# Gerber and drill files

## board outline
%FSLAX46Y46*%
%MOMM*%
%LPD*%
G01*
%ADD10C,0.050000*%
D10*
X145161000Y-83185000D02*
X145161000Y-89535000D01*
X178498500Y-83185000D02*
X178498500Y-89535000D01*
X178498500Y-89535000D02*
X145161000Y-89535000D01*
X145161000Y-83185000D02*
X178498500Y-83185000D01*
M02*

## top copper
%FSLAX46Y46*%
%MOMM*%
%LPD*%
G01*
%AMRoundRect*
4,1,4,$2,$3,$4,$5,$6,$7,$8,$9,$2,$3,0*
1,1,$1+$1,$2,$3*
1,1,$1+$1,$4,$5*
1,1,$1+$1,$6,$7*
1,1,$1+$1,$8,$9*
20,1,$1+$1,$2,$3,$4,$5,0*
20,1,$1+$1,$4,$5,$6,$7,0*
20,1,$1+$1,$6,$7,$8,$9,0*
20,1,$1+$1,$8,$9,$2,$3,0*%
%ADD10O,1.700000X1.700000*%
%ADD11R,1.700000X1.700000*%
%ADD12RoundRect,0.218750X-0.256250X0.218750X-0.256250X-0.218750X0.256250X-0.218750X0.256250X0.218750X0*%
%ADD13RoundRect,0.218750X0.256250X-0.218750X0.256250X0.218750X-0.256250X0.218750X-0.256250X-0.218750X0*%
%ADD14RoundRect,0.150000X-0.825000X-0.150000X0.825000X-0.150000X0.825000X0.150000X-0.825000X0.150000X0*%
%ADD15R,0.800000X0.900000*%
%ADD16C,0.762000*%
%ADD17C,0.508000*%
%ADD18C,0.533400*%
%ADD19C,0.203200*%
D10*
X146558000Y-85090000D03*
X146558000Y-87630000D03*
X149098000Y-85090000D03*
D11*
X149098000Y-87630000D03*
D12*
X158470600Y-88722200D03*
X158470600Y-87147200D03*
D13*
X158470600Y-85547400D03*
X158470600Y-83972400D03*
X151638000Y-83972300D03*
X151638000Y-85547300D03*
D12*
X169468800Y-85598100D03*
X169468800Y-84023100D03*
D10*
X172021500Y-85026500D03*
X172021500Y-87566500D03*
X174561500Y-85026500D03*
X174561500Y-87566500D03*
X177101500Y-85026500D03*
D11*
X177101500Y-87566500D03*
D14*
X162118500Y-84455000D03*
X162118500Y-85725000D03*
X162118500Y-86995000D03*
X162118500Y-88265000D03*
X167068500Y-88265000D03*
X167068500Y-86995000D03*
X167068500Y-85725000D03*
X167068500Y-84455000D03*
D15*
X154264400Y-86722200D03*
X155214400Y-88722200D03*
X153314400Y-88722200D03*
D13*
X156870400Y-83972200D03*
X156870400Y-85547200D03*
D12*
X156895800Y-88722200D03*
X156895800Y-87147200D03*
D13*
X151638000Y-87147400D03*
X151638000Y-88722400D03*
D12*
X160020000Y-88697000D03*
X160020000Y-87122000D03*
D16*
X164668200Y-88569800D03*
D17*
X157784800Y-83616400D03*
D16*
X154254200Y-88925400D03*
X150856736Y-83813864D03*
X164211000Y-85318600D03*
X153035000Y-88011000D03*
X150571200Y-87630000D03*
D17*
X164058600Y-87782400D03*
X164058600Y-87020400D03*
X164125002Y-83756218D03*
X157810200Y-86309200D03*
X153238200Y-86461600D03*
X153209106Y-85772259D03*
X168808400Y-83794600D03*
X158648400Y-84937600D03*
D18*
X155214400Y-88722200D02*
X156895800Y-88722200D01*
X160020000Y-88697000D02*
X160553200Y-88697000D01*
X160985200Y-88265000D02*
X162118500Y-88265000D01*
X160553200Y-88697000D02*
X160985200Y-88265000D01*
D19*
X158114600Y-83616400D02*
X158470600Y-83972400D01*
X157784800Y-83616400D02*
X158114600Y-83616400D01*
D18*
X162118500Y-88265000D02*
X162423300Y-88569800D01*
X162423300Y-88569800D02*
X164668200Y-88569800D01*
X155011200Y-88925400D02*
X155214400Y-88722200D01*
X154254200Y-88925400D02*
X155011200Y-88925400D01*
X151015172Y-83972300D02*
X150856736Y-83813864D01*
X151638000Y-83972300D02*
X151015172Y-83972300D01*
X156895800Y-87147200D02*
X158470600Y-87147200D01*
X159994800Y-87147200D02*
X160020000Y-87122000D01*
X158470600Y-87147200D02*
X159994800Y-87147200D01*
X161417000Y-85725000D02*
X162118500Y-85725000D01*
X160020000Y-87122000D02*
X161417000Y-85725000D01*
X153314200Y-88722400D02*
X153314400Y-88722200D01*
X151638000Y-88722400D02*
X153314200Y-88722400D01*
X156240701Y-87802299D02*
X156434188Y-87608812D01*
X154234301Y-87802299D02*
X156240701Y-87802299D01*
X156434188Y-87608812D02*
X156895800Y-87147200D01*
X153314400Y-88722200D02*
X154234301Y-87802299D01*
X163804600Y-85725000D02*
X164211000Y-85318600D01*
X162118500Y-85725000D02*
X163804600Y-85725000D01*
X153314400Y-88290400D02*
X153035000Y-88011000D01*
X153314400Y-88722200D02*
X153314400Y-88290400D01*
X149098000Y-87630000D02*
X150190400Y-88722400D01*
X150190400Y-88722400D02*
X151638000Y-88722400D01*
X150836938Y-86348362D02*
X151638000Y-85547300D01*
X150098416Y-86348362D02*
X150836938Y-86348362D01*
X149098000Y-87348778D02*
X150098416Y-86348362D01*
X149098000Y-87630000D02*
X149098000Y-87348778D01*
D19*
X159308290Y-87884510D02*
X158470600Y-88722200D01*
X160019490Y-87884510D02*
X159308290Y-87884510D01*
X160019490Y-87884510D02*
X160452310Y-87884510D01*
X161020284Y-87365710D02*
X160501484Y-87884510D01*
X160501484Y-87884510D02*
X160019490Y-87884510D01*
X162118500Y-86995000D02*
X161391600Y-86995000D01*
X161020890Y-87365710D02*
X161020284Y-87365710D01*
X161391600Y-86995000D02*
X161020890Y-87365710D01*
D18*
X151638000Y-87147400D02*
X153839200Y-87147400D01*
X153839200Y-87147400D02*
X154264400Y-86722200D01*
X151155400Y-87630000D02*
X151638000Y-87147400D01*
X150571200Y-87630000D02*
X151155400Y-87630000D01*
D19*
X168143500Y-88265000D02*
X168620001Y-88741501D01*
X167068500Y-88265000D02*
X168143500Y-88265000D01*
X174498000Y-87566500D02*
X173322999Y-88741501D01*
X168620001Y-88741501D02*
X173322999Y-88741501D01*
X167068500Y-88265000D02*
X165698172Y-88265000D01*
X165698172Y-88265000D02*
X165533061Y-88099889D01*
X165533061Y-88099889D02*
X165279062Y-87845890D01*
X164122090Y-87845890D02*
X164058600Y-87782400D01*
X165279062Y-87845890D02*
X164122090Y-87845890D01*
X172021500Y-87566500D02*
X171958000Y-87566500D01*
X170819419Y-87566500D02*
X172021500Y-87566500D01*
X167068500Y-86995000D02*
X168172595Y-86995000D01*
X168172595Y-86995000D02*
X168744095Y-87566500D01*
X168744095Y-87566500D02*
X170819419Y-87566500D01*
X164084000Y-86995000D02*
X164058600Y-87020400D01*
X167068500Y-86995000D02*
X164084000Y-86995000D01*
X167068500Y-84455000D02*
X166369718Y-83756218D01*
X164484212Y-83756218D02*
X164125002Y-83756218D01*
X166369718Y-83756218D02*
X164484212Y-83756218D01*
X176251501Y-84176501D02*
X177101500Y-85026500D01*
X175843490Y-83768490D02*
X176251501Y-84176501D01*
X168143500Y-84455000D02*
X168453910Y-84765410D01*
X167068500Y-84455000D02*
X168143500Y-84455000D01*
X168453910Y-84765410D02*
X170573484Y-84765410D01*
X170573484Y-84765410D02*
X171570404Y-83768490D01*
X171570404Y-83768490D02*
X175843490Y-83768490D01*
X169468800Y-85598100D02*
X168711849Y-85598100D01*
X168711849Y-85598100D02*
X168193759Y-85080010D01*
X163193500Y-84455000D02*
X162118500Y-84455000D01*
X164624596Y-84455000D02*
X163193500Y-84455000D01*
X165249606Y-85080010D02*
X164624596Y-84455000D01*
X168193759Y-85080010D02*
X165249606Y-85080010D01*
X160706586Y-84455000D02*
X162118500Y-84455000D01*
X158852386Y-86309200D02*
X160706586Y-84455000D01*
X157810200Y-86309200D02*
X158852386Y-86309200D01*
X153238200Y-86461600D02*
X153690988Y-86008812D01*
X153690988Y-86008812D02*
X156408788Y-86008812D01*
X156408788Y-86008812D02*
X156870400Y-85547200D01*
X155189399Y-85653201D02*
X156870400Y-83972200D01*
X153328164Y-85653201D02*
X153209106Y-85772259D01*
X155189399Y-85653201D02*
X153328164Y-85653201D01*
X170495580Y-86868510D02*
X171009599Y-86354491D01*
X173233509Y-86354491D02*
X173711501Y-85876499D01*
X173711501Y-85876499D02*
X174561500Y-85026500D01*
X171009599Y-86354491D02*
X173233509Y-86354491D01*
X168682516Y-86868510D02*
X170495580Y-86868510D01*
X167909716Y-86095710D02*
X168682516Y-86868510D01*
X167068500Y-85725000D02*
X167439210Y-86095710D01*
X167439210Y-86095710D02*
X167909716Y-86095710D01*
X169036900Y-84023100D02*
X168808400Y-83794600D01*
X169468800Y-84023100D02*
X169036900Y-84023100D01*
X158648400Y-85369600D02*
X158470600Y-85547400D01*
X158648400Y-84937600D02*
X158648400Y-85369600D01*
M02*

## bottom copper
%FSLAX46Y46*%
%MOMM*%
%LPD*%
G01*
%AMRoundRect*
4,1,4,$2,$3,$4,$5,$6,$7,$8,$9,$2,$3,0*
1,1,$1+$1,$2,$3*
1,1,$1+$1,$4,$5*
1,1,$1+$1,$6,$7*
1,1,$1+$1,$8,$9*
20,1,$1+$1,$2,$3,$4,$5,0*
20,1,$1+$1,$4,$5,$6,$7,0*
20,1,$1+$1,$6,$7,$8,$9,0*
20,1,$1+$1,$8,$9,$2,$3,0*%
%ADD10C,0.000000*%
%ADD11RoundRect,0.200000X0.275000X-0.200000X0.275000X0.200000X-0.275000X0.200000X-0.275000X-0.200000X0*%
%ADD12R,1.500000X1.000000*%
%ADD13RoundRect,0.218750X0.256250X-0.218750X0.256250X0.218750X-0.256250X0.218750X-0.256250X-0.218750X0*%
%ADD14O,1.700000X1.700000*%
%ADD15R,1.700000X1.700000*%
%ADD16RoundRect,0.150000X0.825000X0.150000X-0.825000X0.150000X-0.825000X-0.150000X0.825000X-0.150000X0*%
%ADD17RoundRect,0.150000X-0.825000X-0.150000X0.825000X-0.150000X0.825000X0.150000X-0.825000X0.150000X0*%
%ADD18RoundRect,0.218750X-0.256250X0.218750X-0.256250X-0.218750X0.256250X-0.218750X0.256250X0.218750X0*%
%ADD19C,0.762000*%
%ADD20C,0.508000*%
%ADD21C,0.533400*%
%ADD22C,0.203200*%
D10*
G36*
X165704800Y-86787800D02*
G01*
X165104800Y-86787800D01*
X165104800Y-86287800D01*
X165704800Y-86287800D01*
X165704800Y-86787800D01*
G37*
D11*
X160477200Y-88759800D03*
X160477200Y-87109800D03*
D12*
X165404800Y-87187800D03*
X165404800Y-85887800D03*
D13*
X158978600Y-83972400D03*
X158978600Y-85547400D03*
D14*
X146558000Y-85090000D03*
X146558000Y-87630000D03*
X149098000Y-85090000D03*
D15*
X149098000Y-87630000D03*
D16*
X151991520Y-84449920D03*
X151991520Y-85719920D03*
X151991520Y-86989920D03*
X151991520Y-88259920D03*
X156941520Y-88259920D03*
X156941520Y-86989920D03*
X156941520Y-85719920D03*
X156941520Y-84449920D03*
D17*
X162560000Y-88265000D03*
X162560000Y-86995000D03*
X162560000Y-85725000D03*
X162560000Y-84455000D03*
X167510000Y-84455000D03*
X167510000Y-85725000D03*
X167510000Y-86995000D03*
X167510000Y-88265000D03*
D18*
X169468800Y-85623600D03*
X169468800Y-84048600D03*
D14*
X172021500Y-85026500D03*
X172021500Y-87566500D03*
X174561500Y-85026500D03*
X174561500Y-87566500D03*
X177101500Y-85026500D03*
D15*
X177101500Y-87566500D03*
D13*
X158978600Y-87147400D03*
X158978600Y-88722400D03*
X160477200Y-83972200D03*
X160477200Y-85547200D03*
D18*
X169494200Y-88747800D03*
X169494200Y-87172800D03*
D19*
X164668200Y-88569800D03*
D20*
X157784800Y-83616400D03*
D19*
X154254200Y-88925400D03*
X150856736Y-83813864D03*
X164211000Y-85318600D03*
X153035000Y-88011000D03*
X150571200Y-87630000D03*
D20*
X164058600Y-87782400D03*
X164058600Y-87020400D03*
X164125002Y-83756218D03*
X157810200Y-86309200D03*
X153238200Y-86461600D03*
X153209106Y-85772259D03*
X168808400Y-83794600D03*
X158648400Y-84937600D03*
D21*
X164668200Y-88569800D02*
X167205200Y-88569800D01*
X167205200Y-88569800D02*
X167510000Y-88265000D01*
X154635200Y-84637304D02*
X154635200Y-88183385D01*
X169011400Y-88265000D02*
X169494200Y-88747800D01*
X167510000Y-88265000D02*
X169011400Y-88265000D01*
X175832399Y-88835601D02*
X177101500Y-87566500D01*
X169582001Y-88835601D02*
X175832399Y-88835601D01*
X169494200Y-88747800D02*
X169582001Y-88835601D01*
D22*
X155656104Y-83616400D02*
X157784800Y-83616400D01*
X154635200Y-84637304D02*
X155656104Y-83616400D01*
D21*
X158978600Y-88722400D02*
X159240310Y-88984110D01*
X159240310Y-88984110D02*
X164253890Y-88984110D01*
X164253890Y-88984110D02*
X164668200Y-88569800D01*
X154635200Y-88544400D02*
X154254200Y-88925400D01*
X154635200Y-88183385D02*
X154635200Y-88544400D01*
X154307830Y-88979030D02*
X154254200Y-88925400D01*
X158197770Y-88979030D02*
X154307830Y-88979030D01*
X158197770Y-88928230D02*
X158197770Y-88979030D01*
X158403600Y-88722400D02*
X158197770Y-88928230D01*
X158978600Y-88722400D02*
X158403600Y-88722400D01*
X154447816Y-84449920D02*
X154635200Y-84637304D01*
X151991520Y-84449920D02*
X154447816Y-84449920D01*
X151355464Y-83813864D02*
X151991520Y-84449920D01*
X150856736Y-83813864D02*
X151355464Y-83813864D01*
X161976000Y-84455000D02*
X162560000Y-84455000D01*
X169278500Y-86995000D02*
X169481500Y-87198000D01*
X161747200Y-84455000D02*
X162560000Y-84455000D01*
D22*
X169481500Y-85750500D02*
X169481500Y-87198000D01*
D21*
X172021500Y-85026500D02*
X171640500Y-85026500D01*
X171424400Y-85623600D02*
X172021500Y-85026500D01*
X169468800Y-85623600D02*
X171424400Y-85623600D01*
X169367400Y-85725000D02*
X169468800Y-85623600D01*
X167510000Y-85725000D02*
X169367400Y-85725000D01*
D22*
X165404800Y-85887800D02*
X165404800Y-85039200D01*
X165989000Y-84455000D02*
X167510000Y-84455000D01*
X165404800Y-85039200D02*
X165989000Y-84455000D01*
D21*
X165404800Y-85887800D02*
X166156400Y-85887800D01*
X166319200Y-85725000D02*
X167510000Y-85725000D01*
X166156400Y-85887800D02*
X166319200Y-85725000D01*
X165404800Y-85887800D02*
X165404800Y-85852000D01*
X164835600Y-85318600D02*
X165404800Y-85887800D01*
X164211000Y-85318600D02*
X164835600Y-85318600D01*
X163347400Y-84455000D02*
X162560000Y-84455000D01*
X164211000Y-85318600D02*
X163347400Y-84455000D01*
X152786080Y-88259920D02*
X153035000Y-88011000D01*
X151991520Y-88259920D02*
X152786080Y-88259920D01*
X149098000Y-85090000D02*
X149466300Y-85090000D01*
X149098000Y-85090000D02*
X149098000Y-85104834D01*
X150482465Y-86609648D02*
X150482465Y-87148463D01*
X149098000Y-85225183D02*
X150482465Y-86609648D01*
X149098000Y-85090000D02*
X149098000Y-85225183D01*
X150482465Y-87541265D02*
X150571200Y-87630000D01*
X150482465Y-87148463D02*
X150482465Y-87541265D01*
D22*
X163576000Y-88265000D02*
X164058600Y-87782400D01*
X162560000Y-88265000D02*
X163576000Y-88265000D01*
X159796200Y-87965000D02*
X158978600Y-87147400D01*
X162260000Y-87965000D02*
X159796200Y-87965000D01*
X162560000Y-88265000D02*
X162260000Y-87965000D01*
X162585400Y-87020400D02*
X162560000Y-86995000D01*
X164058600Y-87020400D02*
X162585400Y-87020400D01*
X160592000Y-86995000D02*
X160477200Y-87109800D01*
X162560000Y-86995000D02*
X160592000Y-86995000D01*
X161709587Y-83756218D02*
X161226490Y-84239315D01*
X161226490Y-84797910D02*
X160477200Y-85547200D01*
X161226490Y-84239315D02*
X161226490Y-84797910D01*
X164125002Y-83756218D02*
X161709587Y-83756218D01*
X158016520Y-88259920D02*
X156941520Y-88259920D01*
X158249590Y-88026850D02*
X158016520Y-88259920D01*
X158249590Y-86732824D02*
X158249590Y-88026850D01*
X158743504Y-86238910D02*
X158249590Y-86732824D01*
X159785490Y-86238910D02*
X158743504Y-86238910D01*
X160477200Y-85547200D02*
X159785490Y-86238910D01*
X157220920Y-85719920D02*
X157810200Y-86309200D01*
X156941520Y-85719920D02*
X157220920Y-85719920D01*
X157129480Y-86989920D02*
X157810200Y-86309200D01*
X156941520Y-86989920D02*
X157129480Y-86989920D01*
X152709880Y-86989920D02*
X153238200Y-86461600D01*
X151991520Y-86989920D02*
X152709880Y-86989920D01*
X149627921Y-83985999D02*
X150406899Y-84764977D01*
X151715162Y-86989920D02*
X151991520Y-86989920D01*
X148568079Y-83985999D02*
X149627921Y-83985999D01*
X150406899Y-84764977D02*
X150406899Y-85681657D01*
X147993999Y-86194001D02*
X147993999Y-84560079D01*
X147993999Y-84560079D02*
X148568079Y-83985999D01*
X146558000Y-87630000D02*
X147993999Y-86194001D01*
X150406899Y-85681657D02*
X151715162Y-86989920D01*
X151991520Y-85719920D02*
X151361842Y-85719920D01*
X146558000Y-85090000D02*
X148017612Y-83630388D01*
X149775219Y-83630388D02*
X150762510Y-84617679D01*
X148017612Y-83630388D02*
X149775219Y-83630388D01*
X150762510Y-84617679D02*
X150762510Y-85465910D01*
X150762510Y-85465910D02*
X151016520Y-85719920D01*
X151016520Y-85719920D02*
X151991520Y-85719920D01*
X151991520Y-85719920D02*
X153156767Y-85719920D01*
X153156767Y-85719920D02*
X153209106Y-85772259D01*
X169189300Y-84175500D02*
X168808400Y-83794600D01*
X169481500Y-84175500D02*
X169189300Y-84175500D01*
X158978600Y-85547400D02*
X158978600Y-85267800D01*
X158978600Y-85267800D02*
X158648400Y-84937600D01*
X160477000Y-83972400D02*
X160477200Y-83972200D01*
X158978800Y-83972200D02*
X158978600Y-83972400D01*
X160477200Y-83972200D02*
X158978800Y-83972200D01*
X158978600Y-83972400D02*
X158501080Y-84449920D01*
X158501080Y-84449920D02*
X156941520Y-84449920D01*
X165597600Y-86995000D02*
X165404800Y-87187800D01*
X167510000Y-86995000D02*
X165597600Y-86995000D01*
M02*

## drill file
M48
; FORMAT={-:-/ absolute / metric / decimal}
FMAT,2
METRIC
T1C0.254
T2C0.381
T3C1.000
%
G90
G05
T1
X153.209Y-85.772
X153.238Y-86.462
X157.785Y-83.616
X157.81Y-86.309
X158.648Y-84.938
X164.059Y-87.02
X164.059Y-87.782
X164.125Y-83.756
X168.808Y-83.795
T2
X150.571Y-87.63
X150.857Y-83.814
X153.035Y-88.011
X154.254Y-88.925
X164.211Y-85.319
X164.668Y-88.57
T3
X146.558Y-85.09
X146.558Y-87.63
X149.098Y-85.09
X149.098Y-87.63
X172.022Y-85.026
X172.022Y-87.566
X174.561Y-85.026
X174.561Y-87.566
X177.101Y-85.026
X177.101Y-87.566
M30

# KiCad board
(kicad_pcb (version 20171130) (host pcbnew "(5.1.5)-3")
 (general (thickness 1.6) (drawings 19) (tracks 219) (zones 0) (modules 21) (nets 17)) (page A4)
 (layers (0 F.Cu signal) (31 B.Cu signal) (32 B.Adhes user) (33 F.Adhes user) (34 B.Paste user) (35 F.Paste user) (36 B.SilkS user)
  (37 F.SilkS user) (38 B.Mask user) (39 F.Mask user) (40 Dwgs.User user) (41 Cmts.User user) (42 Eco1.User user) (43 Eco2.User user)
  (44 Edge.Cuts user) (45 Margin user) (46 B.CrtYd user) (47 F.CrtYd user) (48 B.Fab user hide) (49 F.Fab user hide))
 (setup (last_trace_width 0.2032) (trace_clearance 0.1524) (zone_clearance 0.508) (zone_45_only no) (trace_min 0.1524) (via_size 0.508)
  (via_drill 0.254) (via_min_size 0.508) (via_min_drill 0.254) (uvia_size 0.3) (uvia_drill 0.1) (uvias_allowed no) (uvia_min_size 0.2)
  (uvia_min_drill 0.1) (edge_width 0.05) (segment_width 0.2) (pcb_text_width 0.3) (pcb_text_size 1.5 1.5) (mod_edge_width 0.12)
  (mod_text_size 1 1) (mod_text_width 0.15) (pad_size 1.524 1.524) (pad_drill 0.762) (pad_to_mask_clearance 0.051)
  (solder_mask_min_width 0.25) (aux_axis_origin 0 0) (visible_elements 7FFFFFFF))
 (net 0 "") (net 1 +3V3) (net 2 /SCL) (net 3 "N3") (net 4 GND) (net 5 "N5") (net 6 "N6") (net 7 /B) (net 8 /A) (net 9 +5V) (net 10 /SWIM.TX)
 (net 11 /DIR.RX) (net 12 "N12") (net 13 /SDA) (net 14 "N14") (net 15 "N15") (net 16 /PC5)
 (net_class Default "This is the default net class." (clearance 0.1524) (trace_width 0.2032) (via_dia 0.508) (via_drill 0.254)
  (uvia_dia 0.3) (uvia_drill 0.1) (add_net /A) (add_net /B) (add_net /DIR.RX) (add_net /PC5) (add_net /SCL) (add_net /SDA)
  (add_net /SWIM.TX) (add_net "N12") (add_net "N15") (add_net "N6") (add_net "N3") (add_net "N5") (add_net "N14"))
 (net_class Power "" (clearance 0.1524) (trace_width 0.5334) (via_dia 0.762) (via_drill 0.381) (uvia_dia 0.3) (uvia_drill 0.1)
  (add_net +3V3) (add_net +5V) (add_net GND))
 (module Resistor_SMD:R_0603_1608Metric (layer B.Cu) (at 160.4772 87.9348 90)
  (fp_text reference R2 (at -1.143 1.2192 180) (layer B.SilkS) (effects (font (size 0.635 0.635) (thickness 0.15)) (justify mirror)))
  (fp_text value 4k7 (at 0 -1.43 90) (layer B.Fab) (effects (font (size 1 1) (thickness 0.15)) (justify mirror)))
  (pad 1 smd roundrect (at -0.825 0 90) (size 0.8 0.95) (layers B.Cu B.Paste B.Mask) (roundrect_rratio 0.25) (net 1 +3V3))
  (pad 2 smd roundrect (at 0.825 0 90) (size 0.8 0.95) (layers B.Cu B.Paste B.Mask) (roundrect_rratio 0.25) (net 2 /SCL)))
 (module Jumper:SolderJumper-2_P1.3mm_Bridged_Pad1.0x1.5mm (layer B.Cu) (at 165.4048 86.5378 270)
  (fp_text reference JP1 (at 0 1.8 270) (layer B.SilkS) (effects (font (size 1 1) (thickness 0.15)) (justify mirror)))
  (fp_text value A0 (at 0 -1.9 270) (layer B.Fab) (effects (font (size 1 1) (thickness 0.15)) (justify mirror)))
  (fp_poly (pts (xy -0.25 0.3) (xy 0.25 0.3) (xy 0.25 -0.3) (xy -0.25 -0.3)) (layer B.Cu) (width 0))
  (pad 2 smd rect (at 0.65 0 270) (size 1 1.5) (layers B.Cu B.Mask) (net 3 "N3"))
  (pad 1 smd rect (at -0.65 0 270) (size 1 1.5) (layers B.Cu B.Mask) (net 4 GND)))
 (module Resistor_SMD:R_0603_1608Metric (layer B.Cu) (at 158.9786 84.7599 90)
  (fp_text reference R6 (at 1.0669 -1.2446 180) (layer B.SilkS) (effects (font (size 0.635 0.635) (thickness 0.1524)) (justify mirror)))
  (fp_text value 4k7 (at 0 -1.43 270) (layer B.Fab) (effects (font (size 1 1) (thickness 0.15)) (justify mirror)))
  (pad 2 smd roundrect (at 0.7875 0 90) (size 0.875 0.95) (layers B.Cu B.Paste B.Mask) (roundrect_rratio 0.25) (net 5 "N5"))
  (pad 1 smd roundrect (at -0.7875 0 90) (size 0.875 0.95) (layers B.Cu B.Paste B.Mask) (roundrect_rratio 0.25) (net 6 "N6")))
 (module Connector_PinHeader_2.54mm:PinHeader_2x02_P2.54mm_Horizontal (layer B.Cu) (at 149.098 87.63 90)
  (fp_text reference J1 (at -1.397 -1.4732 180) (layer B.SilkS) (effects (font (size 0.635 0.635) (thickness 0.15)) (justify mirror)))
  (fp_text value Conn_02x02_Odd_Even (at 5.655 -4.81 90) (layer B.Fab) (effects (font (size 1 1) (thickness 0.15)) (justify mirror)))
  (pad 4 thru_hole oval (at 2.54 -2.54 90) (size 1.7 1.7) (drill 1) (layers *.Cu *.Mask) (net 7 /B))
  (pad 3 thru_hole oval (at 0 -2.54 90) (size 1.7 1.7) (drill 1) (layers *.Cu *.Mask) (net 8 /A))
  (pad 2 thru_hole oval (at 2.54 0 90) (size 1.7 1.7) (drill 1) (layers *.Cu *.Mask) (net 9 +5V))
  (pad 1 thru_hole rect (at 0 0 90) (size 1.7 1.7) (drill 1) (layers *.Cu *.Mask) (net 4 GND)))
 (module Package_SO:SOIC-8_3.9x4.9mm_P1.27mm (layer B.Cu) (at 154.46652 86.35492 180)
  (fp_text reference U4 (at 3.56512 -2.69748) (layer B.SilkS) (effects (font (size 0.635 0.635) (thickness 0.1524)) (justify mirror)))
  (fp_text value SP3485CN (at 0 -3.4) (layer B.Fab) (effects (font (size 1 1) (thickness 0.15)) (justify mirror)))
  (pad 8 smd roundrect (at 2.475 1.905 180) (size 1.95 0.6) (layers B.Cu B.Paste B.Mask) (roundrect_rratio 0.25) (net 1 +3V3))
  (pad 7 smd roundrect (at 2.475 0.635 180) (size 1.95 0.6) (layers B.Cu B.Paste B.Mask) (roundrect_rratio 0.25) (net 7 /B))
  (pad 6 smd roundrect (at 2.475 -0.635 180) (size 1.95 0.6) (layers B.Cu B.Paste B.Mask) (roundrect_rratio 0.25) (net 8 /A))
  (pad 5 smd roundrect (at 2.475 -1.905 180) (size 1.95 0.6) (layers B.Cu B.Paste B.Mask) (roundrect_rratio 0.25) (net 4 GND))
  (pad 4 smd roundrect (at -2.475 -1.905 180) (size 1.95 0.6) (layers B.Cu B.Paste B.Mask) (roundrect_rratio 0.25) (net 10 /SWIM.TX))
  (pad 3 smd roundrect (at -2.475 -0.635 180) (size 1.95 0.6) (layers B.Cu B.Paste B.Mask) (roundrect_rratio 0.25) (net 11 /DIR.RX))
  (pad 2 smd roundrect (at -2.475 0.635 180) (size 1.95 0.6) (layers B.Cu B.Paste B.Mask) (roundrect_rratio 0.25) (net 11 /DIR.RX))
  (pad 1 smd roundrect (at -2.475 1.905 180) (size 1.95 0.6) (layers B.Cu B.Paste B.Mask) (roundrect_rratio 0.25) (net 5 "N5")))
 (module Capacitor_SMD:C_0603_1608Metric (layer F.Cu) (at 158.4706 87.9347 270)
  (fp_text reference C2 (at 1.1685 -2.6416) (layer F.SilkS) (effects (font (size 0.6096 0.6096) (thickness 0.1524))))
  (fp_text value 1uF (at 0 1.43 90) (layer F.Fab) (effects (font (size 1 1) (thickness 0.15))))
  (pad 2 smd roundrect (at 0.7875 0 270) (size 0.875 0.95) (layers F.Cu F.Paste F.Mask) (roundrect_rratio 0.25) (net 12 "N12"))
  (pad 1 smd roundrect (at -0.7875 0 270) (size 0.875 0.95) (layers F.Cu F.Paste F.Mask) (roundrect_rratio 0.25) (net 4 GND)))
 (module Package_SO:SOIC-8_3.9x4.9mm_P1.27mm (layer B.Cu) (at 165.035 86.36)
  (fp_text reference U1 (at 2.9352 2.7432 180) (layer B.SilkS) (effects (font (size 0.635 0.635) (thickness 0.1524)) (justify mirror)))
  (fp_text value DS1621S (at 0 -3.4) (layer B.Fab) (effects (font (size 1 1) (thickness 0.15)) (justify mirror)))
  (pad 1 smd roundrect (at -2.475 1.905) (size 1.95 0.6) (layers B.Cu B.Paste B.Mask) (roundrect_rratio 0.25) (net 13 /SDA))
  (pad 2 smd roundrect (at -2.475 0.635) (size 1.95 0.6) (layers B.Cu B.Paste B.Mask) (roundrect_rratio 0.25) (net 2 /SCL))
  (pad 3 smd roundrect (at -2.475 -0.635) (size 1.95 0.6) (layers B.Cu B.Paste B.Mask) (roundrect_rratio 0.25) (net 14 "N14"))
  (pad 4 smd roundrect (at -2.475 -1.905) (size 1.95 0.6) (layers B.Cu B.Paste B.Mask) (roundrect_rratio 0.25) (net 4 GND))
  (pad 5 smd roundrect (at 2.475 -1.905) (size 1.95 0.6) (layers B.Cu B.Paste B.Mask) (roundrect_rratio 0.25) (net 4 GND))
  (pad 6 smd roundrect (at 2.475 -0.635) (size 1.95 0.6) (layers B.Cu B.Paste B.Mask) (roundrect_rratio 0.25) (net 4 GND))
  (pad 7 smd roundrect (at 2.475 0.635) (size 1.95 0.6) (layers B.Cu B.Paste B.Mask) (roundrect_rratio 0.25) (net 3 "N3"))
  (pad 8 smd roundrect (at 2.475 1.905) (size 1.95 0.6) (layers B.Cu B.Paste B.Mask) (roundrect_rratio 0.25) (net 1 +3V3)))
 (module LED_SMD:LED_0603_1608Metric (layer F.Cu) (at 158.4706 84.7599 90)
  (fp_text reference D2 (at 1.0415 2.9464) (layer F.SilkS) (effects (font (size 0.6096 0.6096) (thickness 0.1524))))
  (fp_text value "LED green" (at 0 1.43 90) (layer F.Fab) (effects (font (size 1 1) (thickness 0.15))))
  (pad 1 smd roundrect (at -0.7875 0 90) (size 0.875 0.95) (layers F.Cu F.Paste F.Mask) (roundrect_rratio 0.25) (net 6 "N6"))
  (pad 2 smd roundrect (at 0.7875 0 90) (size 0.875 0.95) (layers F.Cu F.Paste F.Mask) (roundrect_rratio 0.25) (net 1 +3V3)))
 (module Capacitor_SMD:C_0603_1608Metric (layer F.Cu) (at 151.638 84.7598 90)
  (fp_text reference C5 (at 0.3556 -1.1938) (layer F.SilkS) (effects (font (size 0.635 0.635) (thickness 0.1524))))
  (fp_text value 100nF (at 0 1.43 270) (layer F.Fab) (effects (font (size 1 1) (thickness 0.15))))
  (pad 2 smd roundrect (at 0.7875 0 90) (size 0.875 0.95) (layers F.Cu F.Paste F.Mask) (roundrect_rratio 0.25) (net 1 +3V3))
  (pad 1 smd roundrect (at -0.7875 0 90) (size 0.875 0.95) (layers F.Cu F.Paste F.Mask) (roundrect_rratio 0.25) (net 4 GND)))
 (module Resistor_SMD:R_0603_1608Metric (layer B.Cu) (at 169.4688 84.8361 270)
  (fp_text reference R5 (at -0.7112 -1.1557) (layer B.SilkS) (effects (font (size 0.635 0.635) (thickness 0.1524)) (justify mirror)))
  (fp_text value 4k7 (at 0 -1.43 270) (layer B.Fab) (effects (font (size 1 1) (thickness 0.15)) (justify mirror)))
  (pad 2 smd roundrect (at 0.7875 0 270) (size 0.875 0.95) (layers B.Cu B.Paste B.Mask) (roundrect_rratio 0.25) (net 4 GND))
  (pad 1 smd roundrect (at -0.7875 0 270) (size 0.875 0.95) (layers B.Cu B.Paste B.Mask) (roundrect_rratio 0.25) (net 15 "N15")))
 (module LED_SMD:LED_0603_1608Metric (layer F.Cu) (at 169.4688 84.8106 270)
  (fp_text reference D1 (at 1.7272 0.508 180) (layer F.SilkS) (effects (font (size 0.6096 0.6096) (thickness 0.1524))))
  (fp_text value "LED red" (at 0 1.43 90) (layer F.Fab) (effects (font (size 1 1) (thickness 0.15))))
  (pad 2 smd roundrect (at 0.7875 0 270) (size 0.875 0.95) (layers F.Cu F.Paste F.Mask) (roundrect_rratio 0.25) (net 11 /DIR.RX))
  (pad 1 smd roundrect (at -0.7875 0 270) (size 0.875 0.95) (layers F.Cu F.Paste F.Mask) (roundrect_rratio 0.25) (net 15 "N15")))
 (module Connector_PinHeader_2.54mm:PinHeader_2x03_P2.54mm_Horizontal (layer B.Cu) (at 177.1015 87.5665 90)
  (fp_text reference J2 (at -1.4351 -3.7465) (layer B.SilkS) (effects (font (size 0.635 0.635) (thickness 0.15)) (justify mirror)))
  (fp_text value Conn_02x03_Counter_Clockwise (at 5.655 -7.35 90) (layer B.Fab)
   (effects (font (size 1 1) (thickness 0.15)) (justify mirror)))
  (pad 6 thru_hole oval (at 2.54 -5.08 90) (size 1.7 1.7) (drill 1) (layers *.Cu *.Mask) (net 4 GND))
  (pad 5 thru_hole oval (at 0 -5.08 90) (size 1.7 1.7) (drill 1) (layers *.Cu *.Mask) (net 2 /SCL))
  (pad 4 thru_hole oval (at 2.54 -2.54 90) (size 1.7 1.7) (drill 1) (layers *.Cu *.Mask) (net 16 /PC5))
  (pad 3 thru_hole oval (at 0 -2.54 90) (size 1.7 1.7) (drill 1) (layers *.Cu *.Mask) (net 13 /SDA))
  (pad 2 thru_hole oval (at 2.54 0 90) (size 1.7 1.7) (drill 1) (layers *.Cu *.Mask) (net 10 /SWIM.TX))
  (pad 1 thru_hole rect (at 0 0 90) (size 1.7 1.7) (drill 1) (layers *.Cu *.Mask) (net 1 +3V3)))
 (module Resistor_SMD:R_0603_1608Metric (layer B.Cu) (at 158.9786 87.9349 90)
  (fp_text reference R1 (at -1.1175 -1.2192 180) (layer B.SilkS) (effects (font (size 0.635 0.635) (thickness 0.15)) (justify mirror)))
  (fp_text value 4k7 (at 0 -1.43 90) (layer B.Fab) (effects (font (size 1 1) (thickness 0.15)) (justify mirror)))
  (pad 2 smd roundrect (at 0.7875 0 90) (size 0.875 0.95) (layers B.Cu B.Paste B.Mask) (roundrect_rratio 0.25) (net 13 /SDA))
  (pad 1 smd roundrect (at -0.7875 0 90) (size 0.875 0.95) (layers B.Cu B.Paste B.Mask) (roundrect_rratio 0.25) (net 1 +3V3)))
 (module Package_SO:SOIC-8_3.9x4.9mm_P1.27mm (layer F.Cu) (at 164.5935 86.36)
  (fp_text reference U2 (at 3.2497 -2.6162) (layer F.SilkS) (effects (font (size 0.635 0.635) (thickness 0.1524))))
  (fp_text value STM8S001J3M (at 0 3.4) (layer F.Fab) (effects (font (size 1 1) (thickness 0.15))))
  (pad 1 smd roundrect (at -2.475 -1.905) (size 1.95 0.6) (layers F.Cu F.Paste F.Mask) (roundrect_rratio 0.25) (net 11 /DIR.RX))
  (pad 2 smd roundrect (at -2.475 -0.635) (size 1.95 0.6) (layers F.Cu F.Paste F.Mask) (roundrect_rratio 0.25) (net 4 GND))
  (pad 3 smd roundrect (at -2.475 0.635) (size 1.95 0.6) (layers F.Cu F.Paste F.Mask) (roundrect_rratio 0.25) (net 12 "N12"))
  (pad 4 smd roundrect (at -2.475 1.905) (size 1.95 0.6) (layers F.Cu F.Paste F.Mask) (roundrect_rratio 0.25) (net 1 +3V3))
  (pad 5 smd roundrect (at 2.475 1.905) (size 1.95 0.6) (layers F.Cu F.Paste F.Mask) (roundrect_rratio 0.25) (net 13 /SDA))
  (pad 6 smd roundrect (at 2.475 0.635) (size 1.95 0.6) (layers F.Cu F.Paste F.Mask) (roundrect_rratio 0.25) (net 2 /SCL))
  (pad 7 smd roundrect (at 2.475 -0.635) (size 1.95 0.6) (layers F.Cu F.Paste F.Mask) (roundrect_rratio 0.25) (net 16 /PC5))
  (pad 8 smd roundrect (at 2.475 -1.905) (size 1.95 0.6) (layers F.Cu F.Paste F.Mask) (roundrect_rratio 0.25) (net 10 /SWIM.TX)))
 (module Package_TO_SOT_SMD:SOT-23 (layer F.Cu) (at 154.2644 87.7222 90)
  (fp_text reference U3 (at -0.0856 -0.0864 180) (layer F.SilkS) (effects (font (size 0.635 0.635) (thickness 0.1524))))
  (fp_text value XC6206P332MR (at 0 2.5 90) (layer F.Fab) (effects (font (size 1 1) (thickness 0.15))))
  (pad 3 smd rect (at 1 0 90) (size 0.9 0.8) (layers F.Cu F.Paste F.Mask) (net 9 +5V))
  (pad 2 smd rect (at -1 0.95 90) (size 0.9 0.8) (layers F.Cu F.Paste F.Mask) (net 1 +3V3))
  (pad 1 smd rect (at -1 -0.95 90) (size 0.9 0.8) (layers F.Cu F.Paste F.Mask) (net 4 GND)))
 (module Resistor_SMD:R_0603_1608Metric (layer F.Cu) (at 156.8704 84.7597 90)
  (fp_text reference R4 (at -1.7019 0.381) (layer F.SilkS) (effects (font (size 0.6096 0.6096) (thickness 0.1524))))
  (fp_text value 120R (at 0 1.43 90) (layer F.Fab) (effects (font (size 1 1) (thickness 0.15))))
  (pad 2 smd roundrect (at 0.7875 0 90) (size 0.875 0.95) (layers F.Cu F.Paste F.Mask) (roundrect_rratio 0.25) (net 7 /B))
  (pad 1 smd roundrect (at -0.7875 0 90) (size 0.875 0.95) (layers F.Cu F.Paste F.Mask) (roundrect_rratio 0.25) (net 8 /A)))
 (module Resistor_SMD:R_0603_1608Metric (layer B.Cu) (at 160.4772 84.7597 90)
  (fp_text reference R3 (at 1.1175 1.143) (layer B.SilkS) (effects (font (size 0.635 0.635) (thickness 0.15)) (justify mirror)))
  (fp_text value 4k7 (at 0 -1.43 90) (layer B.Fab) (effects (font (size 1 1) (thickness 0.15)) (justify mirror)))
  (pad 2 smd roundrect (at 0.7875 0 90) (size 0.875 0.95) (layers B.Cu B.Paste B.Mask) (roundrect_rratio 0.25) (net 5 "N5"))
  (pad 1 smd roundrect (at -0.7875 0 90) (size 0.875 0.95) (layers B.Cu B.Paste B.Mask) (roundrect_rratio 0.25) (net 10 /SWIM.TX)))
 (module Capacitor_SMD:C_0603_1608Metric (layer F.Cu) (at 156.8958 87.9347 270)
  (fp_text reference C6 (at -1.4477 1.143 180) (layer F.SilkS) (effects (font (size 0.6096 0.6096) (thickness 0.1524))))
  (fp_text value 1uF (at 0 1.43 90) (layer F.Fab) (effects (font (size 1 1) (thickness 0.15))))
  (pad 2 smd roundrect (at 0.7875 0 270) (size 0.875 0.95) (layers F.Cu F.Paste F.Mask) (roundrect_rratio 0.25) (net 1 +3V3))
  (pad 1 smd roundrect (at -0.7875 0 270) (size 0.875 0.95) (layers F.Cu F.Paste F.Mask) (roundrect_rratio 0.25) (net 4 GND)))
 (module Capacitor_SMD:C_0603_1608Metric (layer F.Cu) (at 151.638 87.9349 90)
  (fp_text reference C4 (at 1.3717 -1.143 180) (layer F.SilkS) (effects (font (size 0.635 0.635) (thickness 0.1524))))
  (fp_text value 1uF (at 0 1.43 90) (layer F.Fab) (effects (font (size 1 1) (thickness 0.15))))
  (pad 2 smd roundrect (at 0.7875 0 90) (size 0.875 0.95) (layers F.Cu F.Paste F.Mask) (roundrect_rratio 0.25) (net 9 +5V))
  (pad 1 smd roundrect (at -0.7875 0 90) (size 0.875 0.95) (layers F.Cu F.Paste F.Mask) (roundrect_rratio 0.25) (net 4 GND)))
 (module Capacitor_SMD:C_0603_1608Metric (layer F.Cu) (at 160.02 87.9095 270)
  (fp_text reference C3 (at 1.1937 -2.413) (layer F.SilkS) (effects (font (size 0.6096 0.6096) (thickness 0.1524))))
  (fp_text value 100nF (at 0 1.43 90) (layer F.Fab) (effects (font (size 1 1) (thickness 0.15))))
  (pad 2 smd roundrect (at 0.7875 0 270) (size 0.875 0.95) (layers F.Cu F.Paste F.Mask) (roundrect_rratio 0.25) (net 1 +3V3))
  (pad 1 smd roundrect (at -0.7875 0 270) (size 0.875 0.95) (layers F.Cu F.Paste F.Mask) (roundrect_rratio 0.25) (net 4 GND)))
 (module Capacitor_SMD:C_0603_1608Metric (layer B.Cu) (at 169.4942 87.9603 270)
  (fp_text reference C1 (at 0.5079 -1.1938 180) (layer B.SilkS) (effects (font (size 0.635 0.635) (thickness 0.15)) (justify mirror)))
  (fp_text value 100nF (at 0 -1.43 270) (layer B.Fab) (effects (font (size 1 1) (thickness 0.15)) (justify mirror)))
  (pad 2 smd roundrect (at 0.7875 0 270) (size 0.875 0.95) (layers B.Cu B.Paste B.Mask) (roundrect_rratio 0.25) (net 1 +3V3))
  (pad 1 smd roundrect (at -0.7875 0 270) (size 0.875 0.95) (layers B.Cu B.Paste B.Mask) (roundrect_rratio 0.25) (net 4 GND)))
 (gr_line (start 145.161 83.185) (end 145.161 89.535) (layer Edge.Cuts) (width 0.05))
 (gr_line (start 178.4985 83.185) (end 178.4985 89.535) (layer Edge.Cuts) (width 0.05))
 (gr_line (start 178.4985 89.535) (end 145.161 89.535) (layer Edge.Cuts) (width 0.05))
 (gr_line (start 145.161 83.185) (end 178.4985 83.185) (layer Edge.Cuts) (width 0.05))
 (via (at 164.6682 88.5698) (size 0.762) (drill 0.381) (layers F.Cu B.Cu) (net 1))
 (segment (start 164.6682 88.5698) (end 167.2052 88.5698) (width 0.5334) (layer B.Cu) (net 1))
 (segment (start 167.2052 88.5698) (end 167.51 88.265) (width 0.5334) (layer B.Cu) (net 1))
 (segment (start 155.2144 88.7222) (end 156.8958 88.7222) (width 0.5334) (layer F.Cu) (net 1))
 (segment (start 154.6352 84.637304) (end 154.6352 88.183385) (width 0.5334) (layer B.Cu) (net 1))
 (segment (start 169.0114 88.265) (end 169.4942 88.7478) (width 0.5334) (layer B.Cu) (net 1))
 (segment (start 167.51 88.265) (end 169.0114 88.265) (width 0.5334) (layer B.Cu) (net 1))
 (segment (start 175.832399 88.835601) (end 177.1015 87.5665) (width 0.5334) (layer B.Cu) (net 1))
 (segment (start 169.582001 88.835601) (end 175.832399 88.835601) (width 0.5334) (layer B.Cu) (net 1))
 (segment (start 169.4942 88.7478) (end 169.582001 88.835601) (width 0.5334) (layer B.Cu) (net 1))
 (segment (start 160.02 88.697) (end 160.5532 88.697) (width 0.5334) (layer F.Cu) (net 1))
 (segment (start 160.9852 88.265) (end 162.1185 88.265) (width 0.5334) (layer F.Cu) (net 1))
 (segment (start 160.5532 88.697) (end 160.9852 88.265) (width 0.5334) (layer F.Cu) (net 1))
 (segment (start 155.656104 83.6164) (end 157.7848 83.6164) (width 0.2032) (layer B.Cu) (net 1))
 (segment (start 154.6352 84.637304) (end 155.656104 83.6164) (width 0.2032) (layer B.Cu) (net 1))
 (via (at 157.7848 83.6164) (size 0.508) (drill 0.254) (layers F.Cu B.Cu) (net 1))
 (segment (start 158.1146 83.6164) (end 158.4706 83.9724) (width 0.2032) (layer F.Cu) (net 1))
 (segment (start 157.7848 83.6164) (end 158.1146 83.6164) (width 0.2032) (layer F.Cu) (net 1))
 (segment (start 162.1185 88.265) (end 162.4233 88.5698) (width 0.5334) (layer F.Cu) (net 1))
 (segment (start 162.4233 88.5698) (end 164.6682 88.5698) (width 0.5334) (layer F.Cu) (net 1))
 (segment (start 158.9786 88.7224) (end 159.24031 88.98411) (width 0.5334) (layer B.Cu) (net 1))
 (segment (start 159.24031 88.98411) (end 164.25389 88.98411) (width 0.5334) (layer B.Cu) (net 1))
 (segment (start 164.25389 88.98411) (end 164.6682 88.5698) (width 0.5334) (layer B.Cu) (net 1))
 (via (at 154.2542 88.9254) (size 0.762) (drill 0.381) (layers F.Cu B.Cu) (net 1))
 (segment (start 154.6352 88.5444) (end 154.2542 88.9254) (width 0.5334) (layer B.Cu) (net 1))
 (segment (start 154.6352 88.183385) (end 154.6352 88.5444) (width 0.5334) (layer B.Cu) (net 1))
 (segment (start 155.0112 88.9254) (end 155.2144 88.7222) (width 0.5334) (layer F.Cu) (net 1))
 (segment (start 154.2542 88.9254) (end 155.0112 88.9254) (width 0.5334) (layer F.Cu) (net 1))
 (segment (start 154.30783 88.97903) (end 154.2542 88.9254) (width 0.5334) (layer B.Cu) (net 1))
 (segment (start 158.19777 88.97903) (end 154.30783 88.97903) (width 0.5334) (layer B.Cu) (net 1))
 (segment (start 158.19777 88.92823) (end 158.19777 88.97903) (width 0.5334) (layer B.Cu) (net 1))
 (segment (start 158.4036 88.7224) (end 158.19777 88.92823) (width 0.5334) (layer B.Cu) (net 1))
 (segment (start 158.9786 88.7224) (end 158.4036 88.7224) (width 0.5334) (layer B.Cu) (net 1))
 (segment (start 154.447816 84.44992) (end 154.6352 84.637304) (width 0.5334) (layer B.Cu) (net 1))
 (segment (start 151.99152 84.44992) (end 154.447816 84.44992) (width 0.5334) (layer B.Cu) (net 1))
 (via (at 150.856736 83.813864) (size 0.762) (drill 0.381) (layers F.Cu B.Cu) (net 1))
 (segment (start 151.015172 83.9723) (end 150.856736 83.813864) (width 0.5334) (layer F.Cu) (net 1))
 (segment (start 151.638 83.9723) (end 151.015172 83.9723) (width 0.5334) (layer F.Cu) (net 1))
 (segment (start 151.355464 83.813864) (end 151.99152 84.44992) (width 0.5334) (layer B.Cu) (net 1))
 (segment (start 150.856736 83.813864) (end 151.355464 83.813864) (width 0.5334) (layer B.Cu) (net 1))
 (segment (start 161.976 84.455) (end 162.56 84.455) (width 0.5334) (layer B.Cu) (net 4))
 (segment (start 156.8958 87.1472) (end 158.4706 87.1472) (width 0.5334) (layer F.Cu) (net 4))
 (segment (start 159.9948 87.1472) (end 160.02 87.122) (width 0.5334) (layer F.Cu) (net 4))
 (segment (start 158.4706 87.1472) (end 159.9948 87.1472) (width 0.5334) (layer F.Cu) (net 4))
 (segment (start 161.417 85.725) (end 162.1185 85.725) (width 0.5334) (layer F.Cu) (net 4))
 (segment (start 160.02 87.122) (end 161.417 85.725) (width 0.5334) (layer F.Cu) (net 4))
 (segment (start 169.2785 86.995) (end 169.4815 87.198) (width 0.5334) (layer B.Cu) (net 4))
 (segment (start 161.7472 84.455) (end 162.56 84.455) (width 0.5334) (layer B.Cu) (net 4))
 (segment (start 169.4815 85.7505) (end 169.4815 87.198) (width 0.2032) (layer B.Cu) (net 4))
 (segment (start 153.3142 88.7224) (end 153.3144 88.7222) (width 0.5334) (layer F.Cu) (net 4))
 (segment (start 151.638 88.7224) (end 153.3142 88.7224) (width 0.5334) (layer F.Cu) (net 4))
 (segment (start 156.240701 87.802299) (end 156.434188 87.608812) (width 0.5334) (layer F.Cu) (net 4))
 (segment (start 154.234301 87.802299) (end 156.240701 87.802299) (width 0.5334) (layer F.Cu) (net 4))
 (segment (start 156.434188 87.608812) (end 156.8958 87.1472) (width 0.5334) (layer F.Cu) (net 4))
 (segment (start 153.3144 88.7222) (end 154.234301 87.802299) (width 0.5334) (layer F.Cu) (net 4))
 (segment (start 172.0215 85.0265) (end 171.6405 85.0265) (width 0.5334) (layer B.Cu) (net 4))
 (segment (start 171.4244 85.6236) (end 172.0215 85.0265) (width 0.5334) (layer B.Cu) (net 4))
 (segment (start 169.4688 85.6236) (end 171.4244 85.6236) (width 0.5334) (layer B.Cu) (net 4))
 (segment (start 169.3674 85.725) (end 169.4688 85.6236) (width 0.5334) (layer B.Cu) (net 4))
 (segment (start 167.51 85.725) (end 169.3674 85.725) (width 0.5334) (layer B.Cu) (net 4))
 (segment (start 165.4048 85.8878) (end 165.4048 85.0392) (width 0.2032) (layer B.Cu) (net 4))
 (segment (start 165.989 84.455) (end 167.51 84.455) (width 0.2032) (layer B.Cu) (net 4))
 (segment (start 165.4048 85.0392) (end 165.989 84.455) (width 0.2032) (layer B.Cu) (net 4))
 (segment (start 165.4048 85.8878) (end 166.1564 85.8878) (width 0.5334) (layer B.Cu) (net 4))
 (segment (start 166.3192 85.725) (end 167.51 85.725) (width 0.5334) (layer B.Cu) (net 4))
 (segment (start 166.1564 85.8878) (end 166.3192 85.725) (width 0.5334) (layer B.Cu) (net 4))
 (segment (start 165.4048 85.8878) (end 165.4048 85.852) (width 0.5334) (layer B.Cu) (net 4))
 (via (at 164.211 85.3186) (size 0.762) (drill 0.381) (layers F.Cu B.Cu) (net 4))
 (segment (start 163.8046 85.725) (end 164.211 85.3186) (width 0.5334) (layer F.Cu) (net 4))
 (segment (start 162.1185 85.725) (end 163.8046 85.725) (width 0.5334) (layer F.Cu) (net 4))
 (segment (start 164.8356 85.3186) (end 165.4048 85.8878) (width 0.5334) (layer B.Cu) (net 4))
 (segment (start 164.211 85.3186) (end 164.8356 85.3186) (width 0.5334) (layer B.Cu) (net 4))
 (segment (start 163.3474 84.455) (end 162.56 84.455) (width 0.5334) (layer B.Cu) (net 4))
 (segment (start 164.211 85.3186) (end 163.3474 84.455) (width 0.5334) (layer B.Cu) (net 4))
 (via (at 153.035 88.011) (size 0.762) (drill 0.381) (layers F.Cu B.Cu) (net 4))
 (segment (start 153.3144 88.2904) (end 153.035 88.011) (width 0.5334) (layer F.Cu) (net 4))
 (segment (start 153.3144 88.7222) (end 153.3144 88.2904) (width 0.5334) (layer F.Cu) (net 4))
 (segment (start 152.78608 88.25992) (end 153.035 88.011) (width 0.5334) (layer B.Cu) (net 4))
 (segment (start 151.99152 88.25992) (end 152.78608 88.25992) (width 0.5334) (layer B.Cu) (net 4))
 (segment (start 149.098 87.63) (end 150.1904 88.7224) (width 0.5334) (layer F.Cu) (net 4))
 (segment (start 150.1904 88.7224) (end 151.638 88.7224) (width 0.5334) (layer F.Cu) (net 4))
 (segment (start 150.836938 86.348362) (end 151.638 85.5473) (width 0.5334) (layer F.Cu) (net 4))
 (segment (start 150.098416 86.348362) (end 150.836938 86.348362) (width 0.5334) (layer F.Cu) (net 4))
 (segment (start 149.098 87.348778) (end 150.098416 86.348362) (width 0.5334) (layer F.Cu) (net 4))
 (segment (start 149.098 87.63) (end 149.098 87.348778) (width 0.5334) (layer F.Cu) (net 4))
 (segment (start 159.30829 87.88451) (end 158.4706 88.7222) (width 0.2032) (layer F.Cu) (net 12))
 (segment (start 160.01949 87.88451) (end 159.30829 87.88451) (width 0.2032) (layer F.Cu) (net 12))
 (segment (start 160.01949 87.88451) (end 160.45231 87.88451) (width 0.2032) (layer F.Cu) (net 12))
 (segment (start 161.020284 87.36571) (end 160.501484 87.88451) (width 0.2032) (layer F.Cu) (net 12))
 (segment (start 160.501484 87.88451) (end 160.01949 87.88451) (width 0.2032) (layer F.Cu) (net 12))
 (segment (start 162.1185 86.995) (end 161.3916 86.995) (width 0.2032) (layer F.Cu) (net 12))
 (segment (start 161.02089 87.36571) (end 161.020284 87.36571) (width 0.2032) (layer F.Cu) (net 12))
 (segment (start 161.3916 86.995) (end 161.02089 87.36571) (width 0.2032) (layer F.Cu) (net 12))
 (segment (start 151.638 87.1474) (end 153.8392 87.1474) (width 0.5334) (layer F.Cu) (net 9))
 (segment (start 153.8392 87.1474) (end 154.2644 86.7222) (width 0.5334) (layer F.Cu) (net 9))
 (segment (start 149.098 85.09) (end 149.4663 85.09) (width 0.5334) (layer B.Cu) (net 9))
 (segment (start 149.098 85.09) (end 149.098 85.104834) (width 0.5334) (layer B.Cu) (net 9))
 (segment (start 150.482465 86.609648) (end 150.482465 87.148463) (width 0.5334) (layer B.Cu) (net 9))
 (segment (start 149.098 85.225183) (end 150.482465 86.609648) (width 0.5334) (layer B.Cu) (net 9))
 (segment (start 149.098 85.09) (end 149.098 85.225183) (width 0.5334) (layer B.Cu) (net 9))
 (via (at 150.5712 87.63) (size 0.762) (drill 0.381) (layers F.Cu B.Cu) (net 9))
 (segment (start 150.482465 87.541265) (end 150.5712 87.63) (width 0.5334) (layer B.Cu) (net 9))
 (segment (start 150.482465 87.148463) (end 150.482465 87.541265) (width 0.5334) (layer B.Cu) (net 9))
 (segment (start 151.1554 87.63) (end 151.638 87.1474) (width 0.5334) (layer F.Cu) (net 9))
 (segment (start 150.5712 87.63) (end 151.1554 87.63) (width 0.5334) (layer F.Cu) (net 9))
 (segment (start 168.1435 88.265) (end 168.620001 88.741501) (width 0.2032) (layer F.Cu) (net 13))
 (segment (start 167.0685 88.265) (end 168.1435 88.265) (width 0.2032) (layer F.Cu) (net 13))
 (segment (start 174.498 87.5665) (end 173.322999 88.741501) (width 0.2032) (layer F.Cu) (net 13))
 (segment (start 168.620001 88.741501) (end 173.322999 88.741501) (width 0.2032) (layer F.Cu) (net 13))
 (segment (start 167.0685 88.265) (end 165.698172 88.265) (width 0.2032) (layer F.Cu) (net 13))
 (segment (start 165.698172 88.265) (end 165.533061 88.099889) (width 0.2032) (layer F.Cu) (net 13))
 (segment (start 165.533061 88.099889) (end 165.279062 87.84589) (width 0.2032) (layer F.Cu) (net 13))
 (via (at 164.0586 87.7824) (size 0.508) (drill 0.254) (layers F.Cu B.Cu) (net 13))
 (segment (start 164.12209 87.84589) (end 164.0586 87.7824) (width 0.2032) (layer F.Cu) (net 13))
 (segment (start 165.279062 87.84589) (end 164.12209 87.84589) (width 0.2032) (layer F.Cu) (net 13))
 (segment (start 163.576 88.265) (end 164.0586 87.7824) (width 0.2032) (layer B.Cu) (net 13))
 (segment (start 162.56 88.265) (end 163.576 88.265) (width 0.2032) (layer B.Cu) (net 13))
 (segment (start 159.7962 87.965) (end 158.9786 87.1474) (width 0.2032) (layer B.Cu) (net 13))
 (segment (start 162.26 87.965) (end 159.7962 87.965) (width 0.2032) (layer B.Cu) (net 13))
 (segment (start 162.56 88.265) (end 162.26 87.965) (width 0.2032) (layer B.Cu) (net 13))
 (segment (start 172.0215 87.5665) (end 171.958 87.5665) (width 0.2032) (layer F.Cu) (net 2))
 (segment (start 170.819419 87.5665) (end 172.0215 87.5665) (width 0.2032) (layer F.Cu) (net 2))
 (segment (start 167.0685 86.995) (end 168.172595 86.995) (width 0.2032) (layer F.Cu) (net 2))
 (segment (start 168.172595 86.995) (end 168.744095 87.5665) (width 0.2032) (layer F.Cu) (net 2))
 (segment (start 168.744095 87.5665) (end 170.819419 87.5665) (width 0.2032) (layer F.Cu) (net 2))
 (via (at 164.0586 87.0204) (size 0.508) (drill 0.254) (layers F.Cu B.Cu) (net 2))
 (segment (start 164.084 86.995) (end 164.0586 87.0204) (width 0.2032) (layer F.Cu) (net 2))
 (segment (start 167.0685 86.995) (end 164.084 86.995) (width 0.2032) (layer F.Cu) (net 2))
 (segment (start 162.5854 87.0204) (end 162.56 86.995) (width 0.2032) (layer B.Cu) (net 2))
 (segment (start 164.0586 87.0204) (end 162.5854 87.0204) (width 0.2032) (layer B.Cu) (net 2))
 (segment (start 160.592 86.995) (end 160.4772 87.1098) (width 0.2032) (layer B.Cu) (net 2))
 (segment (start 162.56 86.995) (end 160.592 86.995) (width 0.2032) (layer B.Cu) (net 2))
 (via (at 164.125002 83.756218) (size 0.508) (drill 0.254) (layers F.Cu B.Cu) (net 10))
 (segment (start 167.0685 84.455) (end 166.369718 83.756218) (width 0.2032) (layer F.Cu) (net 10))
 (segment (start 164.484212 83.756218) (end 164.125002 83.756218) (width 0.2032) (layer F.Cu) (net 10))
 (segment (start 166.369718 83.756218) (end 164.484212 83.756218) (width 0.2032) (layer F.Cu) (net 10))
 (segment (start 176.251501 84.176501) (end 177.1015 85.0265) (width 0.2032) (layer F.Cu) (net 10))
 (segment (start 175.84349 83.76849) (end 176.251501 84.176501) (width 0.2032) (layer F.Cu) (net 10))
 (segment (start 168.1435 84.455) (end 168.45391 84.76541) (width 0.2032) (layer F.Cu) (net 10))
 (segment (start 167.0685 84.455) (end 168.1435 84.455) (width 0.2032) (layer F.Cu) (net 10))
 (segment (start 168.45391 84.76541) (end 170.573484 84.76541) (width 0.2032) (layer F.Cu) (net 10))
 (segment (start 170.573484 84.76541) (end 171.570404 83.76849) (width 0.2032) (layer F.Cu) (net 10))
 (segment (start 171.570404 83.76849) (end 175.84349 83.76849) (width 0.2032) (layer F.Cu) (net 10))
 (segment (start 161.709587 83.756218) (end 161.22649 84.239315) (width 0.2032) (layer B.Cu) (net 10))
 (segment (start 161.22649 84.79791) (end 160.4772 85.5472) (width 0.2032) (layer B.Cu) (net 10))
 (segment (start 161.22649 84.239315) (end 161.22649 84.79791) (width 0.2032) (layer B.Cu) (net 10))
 (segment (start 164.125002 83.756218) (end 161.709587 83.756218) (width 0.2032) (layer B.Cu) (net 10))
 (segment (start 158.01652 88.25992) (end 156.94152 88.25992) (width 0.2032) (layer B.Cu) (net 10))
 (segment (start 158.24959 88.02685) (end 158.01652 88.25992) (width 0.2032) (layer B.Cu) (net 10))
 (segment (start 158.24959 86.732824) (end 158.24959 88.02685) (width 0.2032) (layer B.Cu) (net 10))
 (segment (start 158.743504 86.23891) (end 158.24959 86.732824) (width 0.2032) (layer B.Cu) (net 10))
 (segment (start 159.78549 86.23891) (end 158.743504 86.23891) (width 0.2032) (layer B.Cu) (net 10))
 (segment (start 160.4772 85.5472) (end 159.78549 86.23891) (width 0.2032) (layer B.Cu) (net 10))
 (segment (start 169.4688 85.5981) (end 168.711849 85.5981) (width 0.2032) (layer F.Cu) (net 11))
 (segment (start 168.711849 85.5981) (end 168.193759 85.08001) (width 0.2032) (layer F.Cu) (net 11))
 (segment (start 163.1935 84.455) (end 162.1185 84.455) (width 0.2032) (layer F.Cu) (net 11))
 (segment (start 164.624596 84.455) (end 163.1935 84.455) (width 0.2032) (layer F.Cu) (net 11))
 (segment (start 165.249606 85.08001) (end 164.624596 84.455) (width 0.2032) (layer F.Cu) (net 11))
 (segment (start 168.193759 85.08001) (end 165.249606 85.08001) (width 0.2032) (layer F.Cu) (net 11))
 (segment (start 157.22092 85.71992) (end 157.8102 86.3092) (width 0.2032) (layer B.Cu) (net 11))
 (via (at 157.8102 86.3092) (size 0.508) (drill 0.254) (layers F.Cu B.Cu) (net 11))
 (segment (start 156.94152 85.71992) (end 157.22092 85.71992) (width 0.2032) (layer B.Cu) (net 11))
 (segment (start 160.706586 84.455) (end 162.1185 84.455) (width 0.2032) (layer F.Cu) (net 11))
 (segment (start 158.852386 86.3092) (end 160.706586 84.455) (width 0.2032) (layer F.Cu) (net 11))
 (segment (start 157.8102 86.3092) (end 158.852386 86.3092) (width 0.2032) (layer F.Cu) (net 11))
 (segment (start 157.12948 86.98992) (end 157.8102 86.3092) (width 0.2032) (layer B.Cu) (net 11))
 (segment (start 156.94152 86.98992) (end 157.12948 86.98992) (width 0.2032) (layer B.Cu) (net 11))
 (via (at 153.2382 86.4616) (size 0.508) (drill 0.254) (layers F.Cu B.Cu) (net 8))
 (segment (start 152.70988 86.98992) (end 153.2382 86.4616) (width 0.2032) (layer B.Cu) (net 8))
 (segment (start 151.99152 86.98992) (end 152.70988 86.98992) (width 0.2032) (layer B.Cu) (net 8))
 (segment (start 149.627921 83.985999) (end 150.406899 84.764977) (width 0.2032) (layer B.Cu) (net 8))
 (segment (start 151.715162 86.98992) (end 151.99152 86.98992) (width 0.2032) (layer B.Cu) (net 8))
 (segment (start 148.568079 83.985999) (end 149.627921 83.985999) (width 0.2032) (layer B.Cu) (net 8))
 (segment (start 150.406899 84.764977) (end 150.406899 85.681657) (width 0.2032) (layer B.Cu) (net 8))
 (segment (start 147.993999 86.194001) (end 147.993999 84.560079) (width 0.2032) (layer B.Cu) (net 8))
 (segment (start 147.993999 84.560079) (end 148.568079 83.985999) (width 0.2032) (layer B.Cu) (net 8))
 (segment (start 146.558 87.63) (end 147.993999 86.194001) (width 0.2032) (layer B.Cu) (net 8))
 (segment (start 150.406899 85.681657) (end 151.715162 86.98992) (width 0.2032) (layer B.Cu) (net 8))
 (segment (start 153.2382 86.4616) (end 153.690988 86.008812) (width 0.2032) (layer F.Cu) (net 8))
 (segment (start 153.690988 86.008812) (end 156.408788 86.008812) (width 0.2032) (layer F.Cu) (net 8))
 (segment (start 156.408788 86.008812) (end 156.8704 85.5472) (width 0.2032) (layer F.Cu) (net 8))
 (segment (start 151.99152 85.71992) (end 151.361842 85.71992) (width 0.2032) (layer B.Cu) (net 7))
 (segment (start 146.558 85.09) (end 148.017612 83.630388) (width 0.2032) (layer B.Cu) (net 7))
 (segment (start 149.775219 83.630388) (end 150.76251 84.617679) (width 0.2032) (layer B.Cu) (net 7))
 (segment (start 148.017612 83.630388) (end 149.775219 83.630388) (width 0.2032) (layer B.Cu) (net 7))
 (segment (start 150.76251 84.617679) (end 150.76251 85.46591) (width 0.2032) (layer B.Cu) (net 7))
 (segment (start 150.76251 85.46591) (end 151.01652 85.71992) (width 0.2032) (layer B.Cu) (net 7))
 (segment (start 151.01652 85.71992) (end 151.99152 85.71992) (width 0.2032) (layer B.Cu) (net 7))
 (segment (start 151.99152 85.71992) (end 153.156767 85.71992) (width 0.2032) (layer B.Cu) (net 7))
 (segment (start 153.156767 85.71992) (end 153.209106 85.772259) (width 0.2032) (layer B.Cu) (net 7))
 (via (at 153.209106 85.772259) (size 0.508) (drill 0.254) (layers F.Cu B.Cu) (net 7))
 (segment (start 155.189399 85.653201) (end 156.8704 83.9722) (width 0.2032) (layer F.Cu) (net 7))
 (segment (start 153.328164 85.653201) (end 153.209106 85.772259) (width 0.2032) (layer F.Cu) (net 7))
 (segment (start 155.189399 85.653201) (end 153.328164 85.653201) (width 0.2032) (layer F.Cu) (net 7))
 (segment (start 170.49558 86.86851) (end 171.009599 86.354491) (width 0.2032) (layer F.Cu) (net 16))
 (segment (start 173.233509 86.354491) (end 173.711501 85.876499) (width 0.2032) (layer F.Cu) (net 16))
 (segment (start 173.711501 85.876499) (end 174.5615 85.0265) (width 0.2032) (layer F.Cu) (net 16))
 (segment (start 171.009599 86.354491) (end 173.233509 86.354491) (width 0.2032) (layer F.Cu) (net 16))
 (segment (start 168.682516 86.86851) (end 170.49558 86.86851) (width 0.2032) (layer F.Cu) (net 16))
 (segment (start 167.909716 86.09571) (end 168.682516 86.86851) (width 0.2032) (layer F.Cu) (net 16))
 (segment (start 167.0685 85.725) (end 167.43921 86.09571) (width 0.2032) (layer F.Cu) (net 16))
 (segment (start 167.43921 86.09571) (end 167.909716 86.09571) (width 0.2032) (layer F.Cu) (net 16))
 (via (at 168.8084 83.7946) (size 0.508) (drill 0.254) (layers F.Cu B.Cu) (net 15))
 (segment (start 169.1893 84.1755) (end 168.8084 83.7946) (width 0.2032) (layer B.Cu) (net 15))
 (segment (start 169.4815 84.1755) (end 169.1893 84.1755) (width 0.2032) (layer B.Cu) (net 15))
 (segment (start 169.0369 84.0231) (end 168.8084 83.7946) (width 0.2032) (layer F.Cu) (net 15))
 (segment (start 169.4688 84.0231) (end 169.0369 84.0231) (width 0.2032) (layer F.Cu) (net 15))
 (segment (start 158.9786 85.5474) (end 158.9786 85.2678) (width 0.2032) (layer B.Cu) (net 6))
 (segment (start 158.6484 85.3696) (end 158.4706 85.5474) (width 0.2032) (layer F.Cu) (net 6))
 (segment (start 158.6484 84.9376) (end 158.6484 85.3696) (width 0.2032) (layer F.Cu) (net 6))
 (segment (start 158.9786 85.2678) (end 158.6484 84.9376) (width 0.2032) (layer B.Cu) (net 6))
 (via (at 158.6484 84.9376) (size 0.508) (drill 0.254) (layers F.Cu B.Cu) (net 6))
 (segment (start 160.477 83.9724) (end 160.4772 83.9722) (width 0.2032) (layer B.Cu) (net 5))
 (segment (start 158.9788 83.9722) (end 158.9786 83.9724) (width 0.2032) (layer B.Cu) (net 5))
 (segment (start 160.4772 83.9722) (end 158.9788 83.9722) (width 0.2032) (layer B.Cu) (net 5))
 (segment (start 158.9786 83.9724) (end 158.50108 84.44992) (width 0.2032) (layer B.Cu) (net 5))
 (segment (start 158.50108 84.44992) (end 156.94152 84.44992) (width 0.2032) (layer B.Cu) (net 5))
 (segment (start 165.5976 86.995) (end 165.4048 87.1878) (width 0.2032) (layer B.Cu) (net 3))
 (segment (start 167.51 86.995) (end 165.5976 86.995) (width 0.2032) (layer B.Cu) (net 3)))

